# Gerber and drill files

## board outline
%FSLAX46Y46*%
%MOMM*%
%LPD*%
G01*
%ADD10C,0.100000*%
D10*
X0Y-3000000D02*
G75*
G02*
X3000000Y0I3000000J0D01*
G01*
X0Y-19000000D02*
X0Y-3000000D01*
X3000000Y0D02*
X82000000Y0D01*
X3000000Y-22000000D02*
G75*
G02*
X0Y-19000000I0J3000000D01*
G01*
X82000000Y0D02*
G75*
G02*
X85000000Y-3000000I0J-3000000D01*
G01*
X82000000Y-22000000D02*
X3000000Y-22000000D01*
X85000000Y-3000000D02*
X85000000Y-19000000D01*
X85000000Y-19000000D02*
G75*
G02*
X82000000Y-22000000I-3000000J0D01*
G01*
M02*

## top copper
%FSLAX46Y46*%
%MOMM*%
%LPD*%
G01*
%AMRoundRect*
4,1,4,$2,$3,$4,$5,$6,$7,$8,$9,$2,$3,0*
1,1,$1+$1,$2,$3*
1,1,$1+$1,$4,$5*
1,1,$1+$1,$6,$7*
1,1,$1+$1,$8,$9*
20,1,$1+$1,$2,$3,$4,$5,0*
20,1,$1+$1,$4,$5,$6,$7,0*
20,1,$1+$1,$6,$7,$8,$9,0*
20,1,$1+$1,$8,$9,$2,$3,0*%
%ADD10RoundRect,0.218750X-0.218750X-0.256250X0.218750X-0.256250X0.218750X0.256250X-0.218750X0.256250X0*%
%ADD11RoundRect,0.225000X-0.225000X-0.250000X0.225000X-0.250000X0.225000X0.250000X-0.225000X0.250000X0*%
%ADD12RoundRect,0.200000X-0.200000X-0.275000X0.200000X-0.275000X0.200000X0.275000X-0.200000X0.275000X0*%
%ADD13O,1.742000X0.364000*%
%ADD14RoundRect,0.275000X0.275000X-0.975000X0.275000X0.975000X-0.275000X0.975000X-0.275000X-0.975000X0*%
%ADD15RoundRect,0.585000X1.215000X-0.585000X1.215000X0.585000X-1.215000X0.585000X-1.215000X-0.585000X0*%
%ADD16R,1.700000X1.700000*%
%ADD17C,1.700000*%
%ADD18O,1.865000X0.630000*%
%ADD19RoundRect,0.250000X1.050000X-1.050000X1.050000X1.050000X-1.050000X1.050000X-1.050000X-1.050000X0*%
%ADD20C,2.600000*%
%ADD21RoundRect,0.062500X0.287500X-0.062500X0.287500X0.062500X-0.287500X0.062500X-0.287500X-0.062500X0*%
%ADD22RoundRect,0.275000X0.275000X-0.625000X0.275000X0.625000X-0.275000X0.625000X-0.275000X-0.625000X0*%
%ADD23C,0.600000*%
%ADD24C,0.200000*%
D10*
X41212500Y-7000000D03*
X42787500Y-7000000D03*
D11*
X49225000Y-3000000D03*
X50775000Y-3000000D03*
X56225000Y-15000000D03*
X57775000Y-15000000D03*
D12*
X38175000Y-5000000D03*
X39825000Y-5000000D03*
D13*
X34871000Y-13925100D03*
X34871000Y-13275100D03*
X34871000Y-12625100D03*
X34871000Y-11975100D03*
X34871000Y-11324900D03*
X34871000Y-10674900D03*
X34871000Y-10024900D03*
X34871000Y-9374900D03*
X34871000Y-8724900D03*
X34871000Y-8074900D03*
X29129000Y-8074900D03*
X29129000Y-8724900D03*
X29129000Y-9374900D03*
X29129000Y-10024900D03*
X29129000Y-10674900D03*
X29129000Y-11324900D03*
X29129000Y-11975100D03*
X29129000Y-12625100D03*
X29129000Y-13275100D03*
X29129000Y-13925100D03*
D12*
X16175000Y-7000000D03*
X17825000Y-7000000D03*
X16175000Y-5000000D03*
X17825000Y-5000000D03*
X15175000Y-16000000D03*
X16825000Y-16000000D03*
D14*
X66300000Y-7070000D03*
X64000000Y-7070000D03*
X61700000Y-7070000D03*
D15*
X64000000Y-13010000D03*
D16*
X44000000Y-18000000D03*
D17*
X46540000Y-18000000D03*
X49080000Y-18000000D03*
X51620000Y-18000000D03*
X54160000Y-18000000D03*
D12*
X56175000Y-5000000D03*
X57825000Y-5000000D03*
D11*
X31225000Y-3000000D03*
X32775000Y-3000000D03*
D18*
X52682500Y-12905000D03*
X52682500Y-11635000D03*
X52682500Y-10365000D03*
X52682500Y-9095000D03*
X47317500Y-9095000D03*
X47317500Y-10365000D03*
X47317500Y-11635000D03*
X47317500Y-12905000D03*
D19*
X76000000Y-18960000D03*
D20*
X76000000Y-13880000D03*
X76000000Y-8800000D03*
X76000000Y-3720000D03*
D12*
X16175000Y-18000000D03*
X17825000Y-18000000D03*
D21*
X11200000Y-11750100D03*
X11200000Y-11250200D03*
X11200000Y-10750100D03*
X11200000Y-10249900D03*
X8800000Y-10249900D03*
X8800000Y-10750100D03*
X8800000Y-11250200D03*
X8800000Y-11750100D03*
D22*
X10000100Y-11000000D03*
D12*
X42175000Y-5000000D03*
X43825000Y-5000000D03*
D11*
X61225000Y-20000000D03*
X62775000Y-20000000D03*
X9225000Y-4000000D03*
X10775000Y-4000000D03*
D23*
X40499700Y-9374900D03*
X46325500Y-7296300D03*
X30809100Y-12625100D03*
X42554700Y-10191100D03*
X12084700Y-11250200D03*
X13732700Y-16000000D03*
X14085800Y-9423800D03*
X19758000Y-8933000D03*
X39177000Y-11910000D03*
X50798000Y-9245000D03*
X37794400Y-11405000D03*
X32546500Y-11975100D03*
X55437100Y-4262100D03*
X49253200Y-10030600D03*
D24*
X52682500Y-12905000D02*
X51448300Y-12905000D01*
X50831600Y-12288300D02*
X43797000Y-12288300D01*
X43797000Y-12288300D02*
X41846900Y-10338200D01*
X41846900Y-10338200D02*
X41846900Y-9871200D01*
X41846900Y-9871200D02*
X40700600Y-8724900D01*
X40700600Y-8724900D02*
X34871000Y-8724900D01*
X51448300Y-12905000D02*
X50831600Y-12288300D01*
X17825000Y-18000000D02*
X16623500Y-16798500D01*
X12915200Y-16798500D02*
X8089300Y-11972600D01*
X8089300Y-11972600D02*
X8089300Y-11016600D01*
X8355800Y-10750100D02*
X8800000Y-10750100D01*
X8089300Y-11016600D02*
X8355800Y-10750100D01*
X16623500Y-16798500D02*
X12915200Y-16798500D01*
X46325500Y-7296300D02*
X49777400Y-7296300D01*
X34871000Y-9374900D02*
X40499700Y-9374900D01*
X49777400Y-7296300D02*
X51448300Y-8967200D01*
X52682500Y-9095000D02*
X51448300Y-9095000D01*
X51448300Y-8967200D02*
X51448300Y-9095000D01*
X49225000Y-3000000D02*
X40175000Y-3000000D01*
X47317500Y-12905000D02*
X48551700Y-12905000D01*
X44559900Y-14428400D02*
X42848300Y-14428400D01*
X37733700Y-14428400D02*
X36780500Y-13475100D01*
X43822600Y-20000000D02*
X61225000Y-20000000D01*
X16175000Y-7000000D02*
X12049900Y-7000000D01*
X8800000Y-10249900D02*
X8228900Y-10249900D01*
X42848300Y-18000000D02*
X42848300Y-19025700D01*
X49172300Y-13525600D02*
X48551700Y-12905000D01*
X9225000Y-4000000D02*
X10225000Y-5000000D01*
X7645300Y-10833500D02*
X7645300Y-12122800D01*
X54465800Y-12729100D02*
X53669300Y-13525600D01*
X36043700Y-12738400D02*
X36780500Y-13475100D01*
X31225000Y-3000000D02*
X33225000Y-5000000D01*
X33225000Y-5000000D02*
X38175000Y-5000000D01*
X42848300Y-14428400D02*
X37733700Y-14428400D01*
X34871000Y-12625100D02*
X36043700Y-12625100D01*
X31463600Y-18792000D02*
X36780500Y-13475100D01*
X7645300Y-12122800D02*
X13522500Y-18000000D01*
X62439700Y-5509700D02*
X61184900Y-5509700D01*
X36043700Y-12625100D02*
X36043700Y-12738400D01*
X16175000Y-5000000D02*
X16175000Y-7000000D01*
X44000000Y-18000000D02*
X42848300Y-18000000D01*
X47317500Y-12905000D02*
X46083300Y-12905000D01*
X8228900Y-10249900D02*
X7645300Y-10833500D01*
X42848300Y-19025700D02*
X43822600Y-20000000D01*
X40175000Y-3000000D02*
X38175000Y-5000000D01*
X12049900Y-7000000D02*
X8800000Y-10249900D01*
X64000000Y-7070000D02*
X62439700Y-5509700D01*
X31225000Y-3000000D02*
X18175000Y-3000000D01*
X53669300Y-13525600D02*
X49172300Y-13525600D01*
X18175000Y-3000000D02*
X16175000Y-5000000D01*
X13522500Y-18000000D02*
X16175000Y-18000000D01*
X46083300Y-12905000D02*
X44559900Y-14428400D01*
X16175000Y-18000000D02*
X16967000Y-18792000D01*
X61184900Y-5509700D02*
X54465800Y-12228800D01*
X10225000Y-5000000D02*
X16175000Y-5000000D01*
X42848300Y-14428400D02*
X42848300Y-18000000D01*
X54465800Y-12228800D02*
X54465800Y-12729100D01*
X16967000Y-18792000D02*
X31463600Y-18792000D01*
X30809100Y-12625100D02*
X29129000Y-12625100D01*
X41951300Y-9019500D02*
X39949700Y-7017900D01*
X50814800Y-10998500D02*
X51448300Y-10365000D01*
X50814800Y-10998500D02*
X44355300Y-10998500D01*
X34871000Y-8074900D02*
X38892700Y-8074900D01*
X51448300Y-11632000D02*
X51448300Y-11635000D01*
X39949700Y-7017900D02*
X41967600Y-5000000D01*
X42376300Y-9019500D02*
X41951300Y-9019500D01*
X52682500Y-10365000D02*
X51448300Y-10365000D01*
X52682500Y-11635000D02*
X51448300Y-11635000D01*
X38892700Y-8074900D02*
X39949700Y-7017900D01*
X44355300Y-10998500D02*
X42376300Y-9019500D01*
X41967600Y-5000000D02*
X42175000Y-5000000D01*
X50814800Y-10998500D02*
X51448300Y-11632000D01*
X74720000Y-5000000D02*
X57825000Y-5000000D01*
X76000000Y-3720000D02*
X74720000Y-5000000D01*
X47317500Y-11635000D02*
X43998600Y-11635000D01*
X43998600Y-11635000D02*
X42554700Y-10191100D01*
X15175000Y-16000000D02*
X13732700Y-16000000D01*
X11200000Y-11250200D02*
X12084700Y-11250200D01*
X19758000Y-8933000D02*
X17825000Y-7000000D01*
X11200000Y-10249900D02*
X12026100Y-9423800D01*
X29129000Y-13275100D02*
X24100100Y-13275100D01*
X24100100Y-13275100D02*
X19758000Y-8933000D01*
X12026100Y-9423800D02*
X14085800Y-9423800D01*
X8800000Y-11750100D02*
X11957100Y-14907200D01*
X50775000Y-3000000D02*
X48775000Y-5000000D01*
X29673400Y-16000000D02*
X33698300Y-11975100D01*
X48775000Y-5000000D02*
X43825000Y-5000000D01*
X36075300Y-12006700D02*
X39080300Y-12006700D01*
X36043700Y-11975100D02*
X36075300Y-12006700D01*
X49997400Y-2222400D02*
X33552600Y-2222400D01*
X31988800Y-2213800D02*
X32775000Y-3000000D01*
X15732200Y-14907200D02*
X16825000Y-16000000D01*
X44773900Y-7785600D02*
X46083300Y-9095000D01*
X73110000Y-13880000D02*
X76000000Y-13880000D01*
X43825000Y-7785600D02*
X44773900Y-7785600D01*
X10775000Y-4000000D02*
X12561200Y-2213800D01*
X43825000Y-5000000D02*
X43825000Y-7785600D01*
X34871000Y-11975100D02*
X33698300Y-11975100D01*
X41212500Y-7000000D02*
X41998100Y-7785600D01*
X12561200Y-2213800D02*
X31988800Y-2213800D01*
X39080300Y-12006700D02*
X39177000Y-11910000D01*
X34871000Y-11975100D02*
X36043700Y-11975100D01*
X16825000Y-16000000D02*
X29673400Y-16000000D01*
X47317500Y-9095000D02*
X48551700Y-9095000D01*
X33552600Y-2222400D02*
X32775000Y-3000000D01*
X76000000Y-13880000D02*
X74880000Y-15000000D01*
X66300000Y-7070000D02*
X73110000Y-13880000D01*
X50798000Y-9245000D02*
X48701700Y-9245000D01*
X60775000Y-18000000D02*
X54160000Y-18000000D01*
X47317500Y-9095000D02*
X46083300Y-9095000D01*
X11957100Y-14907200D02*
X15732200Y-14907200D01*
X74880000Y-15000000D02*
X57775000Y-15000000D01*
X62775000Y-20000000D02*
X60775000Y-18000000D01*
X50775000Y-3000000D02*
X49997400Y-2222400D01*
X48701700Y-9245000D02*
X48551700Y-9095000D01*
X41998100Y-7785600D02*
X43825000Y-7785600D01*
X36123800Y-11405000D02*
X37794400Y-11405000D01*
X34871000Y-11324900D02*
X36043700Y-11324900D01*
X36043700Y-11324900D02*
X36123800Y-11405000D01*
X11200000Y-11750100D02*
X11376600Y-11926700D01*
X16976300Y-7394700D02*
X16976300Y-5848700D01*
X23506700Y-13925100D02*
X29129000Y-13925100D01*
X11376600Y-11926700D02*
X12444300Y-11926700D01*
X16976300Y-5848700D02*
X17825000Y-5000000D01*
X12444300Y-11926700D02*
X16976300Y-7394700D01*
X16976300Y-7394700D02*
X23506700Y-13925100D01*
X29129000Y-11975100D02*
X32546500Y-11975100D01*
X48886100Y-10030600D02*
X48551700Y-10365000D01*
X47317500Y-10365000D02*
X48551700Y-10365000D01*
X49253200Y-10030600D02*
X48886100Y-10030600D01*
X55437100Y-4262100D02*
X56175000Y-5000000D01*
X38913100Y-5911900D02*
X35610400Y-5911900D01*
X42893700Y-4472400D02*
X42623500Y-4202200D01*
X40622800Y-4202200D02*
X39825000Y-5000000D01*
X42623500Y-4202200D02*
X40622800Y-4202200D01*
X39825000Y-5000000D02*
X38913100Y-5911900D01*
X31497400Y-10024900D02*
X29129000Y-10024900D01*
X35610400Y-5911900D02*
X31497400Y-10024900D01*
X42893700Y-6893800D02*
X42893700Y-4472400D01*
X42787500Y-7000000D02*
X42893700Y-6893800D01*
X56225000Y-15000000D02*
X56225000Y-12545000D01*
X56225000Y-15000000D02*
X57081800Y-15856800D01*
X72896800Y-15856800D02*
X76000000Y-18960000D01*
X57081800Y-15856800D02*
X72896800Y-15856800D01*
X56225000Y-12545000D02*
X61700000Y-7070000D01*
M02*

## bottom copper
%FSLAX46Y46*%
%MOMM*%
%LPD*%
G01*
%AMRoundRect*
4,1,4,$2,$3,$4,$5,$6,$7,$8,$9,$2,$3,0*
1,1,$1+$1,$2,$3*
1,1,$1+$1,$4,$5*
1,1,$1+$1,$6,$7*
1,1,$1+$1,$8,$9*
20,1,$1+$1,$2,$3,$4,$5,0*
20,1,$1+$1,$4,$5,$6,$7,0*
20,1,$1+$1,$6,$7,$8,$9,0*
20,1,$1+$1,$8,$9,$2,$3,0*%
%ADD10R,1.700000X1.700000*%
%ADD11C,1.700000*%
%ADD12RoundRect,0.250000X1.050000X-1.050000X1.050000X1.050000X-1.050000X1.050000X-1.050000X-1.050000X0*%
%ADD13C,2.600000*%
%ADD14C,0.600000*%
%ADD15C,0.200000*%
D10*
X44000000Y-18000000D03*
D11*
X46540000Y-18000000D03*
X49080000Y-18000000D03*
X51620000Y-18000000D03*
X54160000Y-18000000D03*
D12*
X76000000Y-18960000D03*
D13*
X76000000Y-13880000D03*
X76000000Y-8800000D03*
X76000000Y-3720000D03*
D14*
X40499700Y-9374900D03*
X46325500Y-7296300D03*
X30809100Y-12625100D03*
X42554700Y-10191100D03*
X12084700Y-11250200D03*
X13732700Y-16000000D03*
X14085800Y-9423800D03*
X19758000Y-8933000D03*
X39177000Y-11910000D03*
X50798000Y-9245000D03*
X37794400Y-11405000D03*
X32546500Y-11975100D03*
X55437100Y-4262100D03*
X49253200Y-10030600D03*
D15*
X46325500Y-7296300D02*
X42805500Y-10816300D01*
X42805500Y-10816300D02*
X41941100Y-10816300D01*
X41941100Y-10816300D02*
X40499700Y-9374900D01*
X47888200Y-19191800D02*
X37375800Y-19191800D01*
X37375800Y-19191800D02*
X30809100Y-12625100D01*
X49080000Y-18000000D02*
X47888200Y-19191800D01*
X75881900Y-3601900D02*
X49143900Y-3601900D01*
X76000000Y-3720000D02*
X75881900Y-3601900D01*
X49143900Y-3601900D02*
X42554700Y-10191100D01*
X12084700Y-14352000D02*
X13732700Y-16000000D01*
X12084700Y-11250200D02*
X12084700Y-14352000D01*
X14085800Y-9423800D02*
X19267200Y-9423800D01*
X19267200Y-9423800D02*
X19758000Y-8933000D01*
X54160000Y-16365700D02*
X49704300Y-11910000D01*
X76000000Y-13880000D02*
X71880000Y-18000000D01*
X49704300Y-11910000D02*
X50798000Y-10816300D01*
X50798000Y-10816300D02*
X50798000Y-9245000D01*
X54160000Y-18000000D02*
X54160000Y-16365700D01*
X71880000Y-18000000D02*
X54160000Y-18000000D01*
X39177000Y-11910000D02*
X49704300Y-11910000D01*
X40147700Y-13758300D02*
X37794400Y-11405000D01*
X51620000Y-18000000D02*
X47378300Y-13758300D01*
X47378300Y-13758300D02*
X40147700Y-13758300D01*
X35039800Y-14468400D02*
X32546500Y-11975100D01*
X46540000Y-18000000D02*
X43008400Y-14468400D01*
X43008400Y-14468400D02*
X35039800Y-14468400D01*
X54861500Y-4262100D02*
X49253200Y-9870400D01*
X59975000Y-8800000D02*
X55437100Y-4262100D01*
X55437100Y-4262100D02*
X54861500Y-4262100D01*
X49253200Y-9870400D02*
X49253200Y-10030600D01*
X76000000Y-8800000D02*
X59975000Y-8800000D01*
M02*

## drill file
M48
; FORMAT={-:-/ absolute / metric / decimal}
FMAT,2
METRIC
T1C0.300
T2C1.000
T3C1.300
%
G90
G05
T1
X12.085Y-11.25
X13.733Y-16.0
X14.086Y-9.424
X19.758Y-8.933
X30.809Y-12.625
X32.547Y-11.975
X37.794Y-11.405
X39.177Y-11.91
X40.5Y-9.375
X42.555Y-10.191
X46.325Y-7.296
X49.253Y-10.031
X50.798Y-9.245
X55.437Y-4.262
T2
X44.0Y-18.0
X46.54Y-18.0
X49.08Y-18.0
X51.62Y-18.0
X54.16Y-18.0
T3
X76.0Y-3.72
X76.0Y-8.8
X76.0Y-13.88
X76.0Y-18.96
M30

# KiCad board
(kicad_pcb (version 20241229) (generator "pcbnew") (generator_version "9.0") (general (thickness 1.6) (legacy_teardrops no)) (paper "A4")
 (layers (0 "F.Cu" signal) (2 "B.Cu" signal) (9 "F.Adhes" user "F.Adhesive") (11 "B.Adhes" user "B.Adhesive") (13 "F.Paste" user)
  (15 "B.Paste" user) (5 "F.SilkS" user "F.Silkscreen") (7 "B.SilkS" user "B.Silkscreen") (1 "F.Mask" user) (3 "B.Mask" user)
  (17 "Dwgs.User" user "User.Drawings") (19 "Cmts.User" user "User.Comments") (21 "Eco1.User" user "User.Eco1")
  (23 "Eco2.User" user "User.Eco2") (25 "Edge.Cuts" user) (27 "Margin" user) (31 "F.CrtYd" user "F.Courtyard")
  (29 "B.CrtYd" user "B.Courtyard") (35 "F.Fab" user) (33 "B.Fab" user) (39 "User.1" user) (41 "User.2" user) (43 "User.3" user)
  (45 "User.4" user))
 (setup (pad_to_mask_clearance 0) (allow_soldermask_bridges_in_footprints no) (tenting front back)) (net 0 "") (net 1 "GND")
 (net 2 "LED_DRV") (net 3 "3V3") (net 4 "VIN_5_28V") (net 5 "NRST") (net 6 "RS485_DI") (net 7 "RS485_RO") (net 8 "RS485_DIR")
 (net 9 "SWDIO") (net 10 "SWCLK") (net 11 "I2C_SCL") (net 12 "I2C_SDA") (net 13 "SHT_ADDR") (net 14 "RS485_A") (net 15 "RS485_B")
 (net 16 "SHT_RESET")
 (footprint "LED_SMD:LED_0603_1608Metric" (layer "F.Cu") (at 42 7)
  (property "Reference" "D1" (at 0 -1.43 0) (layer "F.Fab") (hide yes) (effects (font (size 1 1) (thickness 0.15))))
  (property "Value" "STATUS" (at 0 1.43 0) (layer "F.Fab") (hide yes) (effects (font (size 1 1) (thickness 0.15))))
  (pad "1" smd roundrect (at -0.7875 0) (size 0.875 0.95) (layers "F.Cu" "F.Mask" "F.Paste") (roundrect_rratio 0.25) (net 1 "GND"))
  (pad "2" smd roundrect (at 0.7875 0) (size 0.875 0.95) (layers "F.Cu" "F.Mask" "F.Paste") (roundrect_rratio 0.25) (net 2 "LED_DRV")))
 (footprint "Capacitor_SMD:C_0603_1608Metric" (layer "F.Cu") (at 50 3)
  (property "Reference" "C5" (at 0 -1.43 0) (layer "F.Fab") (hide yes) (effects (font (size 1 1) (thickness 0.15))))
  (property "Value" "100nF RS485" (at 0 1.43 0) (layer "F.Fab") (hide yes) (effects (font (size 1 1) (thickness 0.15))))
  (pad "1" smd roundrect (at -0.775 0) (size 0.9 0.95) (layers "F.Cu" "F.Mask" "F.Paste") (roundrect_rratio 0.25) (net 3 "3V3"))
  (pad "2" smd roundrect (at 0.775 0) (size 0.9 0.95) (layers "F.Cu" "F.Mask" "F.Paste") (roundrect_rratio 0.25) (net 1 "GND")))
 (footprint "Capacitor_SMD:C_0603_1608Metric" (layer "F.Cu") (at 57 15)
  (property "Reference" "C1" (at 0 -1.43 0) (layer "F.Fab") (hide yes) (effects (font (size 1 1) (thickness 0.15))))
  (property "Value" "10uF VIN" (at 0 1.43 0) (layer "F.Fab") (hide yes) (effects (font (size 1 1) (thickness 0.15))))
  (pad "1" smd roundrect (at -0.775 0) (size 0.9 0.95) (layers "F.Cu" "F.Mask" "F.Paste") (roundrect_rratio 0.25) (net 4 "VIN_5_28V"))
  (pad "2" smd roundrect (at 0.775 0) (size 0.9 0.95) (layers "F.Cu" "F.Mask" "F.Paste") (roundrect_rratio 0.25) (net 1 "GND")))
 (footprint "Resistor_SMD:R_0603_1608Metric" (layer "F.Cu") (at 39 5)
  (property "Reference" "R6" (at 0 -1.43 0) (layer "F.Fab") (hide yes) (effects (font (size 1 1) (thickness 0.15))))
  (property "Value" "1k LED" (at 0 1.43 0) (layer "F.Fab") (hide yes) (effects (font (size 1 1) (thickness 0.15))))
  (pad "1" smd roundrect (at -0.825 0) (size 0.8 0.95) (layers "F.Cu" "F.Mask" "F.Paste") (roundrect_rratio 0.25) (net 3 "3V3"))
  (pad "2" smd roundrect (at 0.825 0) (size 0.8 0.95) (layers "F.Cu" "F.Mask" "F.Paste") (roundrect_rratio 0.25) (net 2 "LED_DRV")))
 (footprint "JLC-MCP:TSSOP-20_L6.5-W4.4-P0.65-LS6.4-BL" (layer "F.Cu") (at 32 11 90)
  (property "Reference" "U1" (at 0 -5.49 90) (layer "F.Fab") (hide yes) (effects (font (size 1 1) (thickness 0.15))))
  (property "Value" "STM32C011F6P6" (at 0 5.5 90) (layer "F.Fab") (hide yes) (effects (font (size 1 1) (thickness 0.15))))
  (pad "1" smd oval (at -2.9251 2.871 90) (size 0.364 1.742) (layers "F.Cu" "F.Mask" "F.Paste"))
  (pad "2" smd oval (at -2.2751 2.871 90) (size 0.364 1.742) (layers "F.Cu" "F.Mask" "F.Paste"))
  (pad "3" smd oval (at -1.6251 2.871 90) (size 0.364 1.742) (layers "F.Cu" "F.Mask" "F.Paste") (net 3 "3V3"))
  (pad "4" smd oval (at -0.9751 2.871 90) (size 0.364 1.742) (layers "F.Cu" "F.Mask" "F.Paste") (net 1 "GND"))
  (pad "5" smd oval (at -0.3249 2.871 90) (size 0.364 1.742) (layers "F.Cu" "F.Mask" "F.Paste") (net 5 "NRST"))
  (pad "6" smd oval (at 0.3251 2.871 90) (size 0.364 1.742) (layers "F.Cu" "F.Mask" "F.Paste"))
  (pad "7" smd oval (at 0.9751 2.871 90) (size 0.364 1.742) (layers "F.Cu" "F.Mask" "F.Paste"))
  (pad "8" smd oval (at 1.6251 2.871 90) (size 0.364 1.742) (layers "F.Cu" "F.Mask" "F.Paste") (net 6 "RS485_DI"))
  (pad "9" smd oval (at 2.2751 2.871 90) (size 0.364 1.742) (layers "F.Cu" "F.Mask" "F.Paste") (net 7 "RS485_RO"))
  (pad "10" smd oval (at 2.9251 2.871 90) (size 0.364 1.742) (layers "F.Cu" "F.Mask" "F.Paste") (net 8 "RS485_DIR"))
  (pad "11" smd oval (at 2.9251 -2.871 90) (size 0.364 1.742) (layers "F.Cu" "F.Mask" "F.Paste"))
  (pad "12" smd oval (at 2.2751 -2.871 90) (size 0.364 1.742) (layers "F.Cu" "F.Mask" "F.Paste"))
  (pad "13" smd oval (at 1.6251 -2.871 90) (size 0.364 1.742) (layers "F.Cu" "F.Mask" "F.Paste"))
  (pad "14" smd oval (at 0.9751 -2.871 90) (size 0.364 1.742) (layers "F.Cu" "F.Mask" "F.Paste") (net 2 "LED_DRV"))
  (pad "15" smd oval (at 0.3251 -2.871 90) (size 0.364 1.742) (layers "F.Cu" "F.Mask" "F.Paste"))
  (pad "16" smd oval (at -0.3249 -2.871 90) (size 0.364 1.742) (layers "F.Cu" "F.Mask" "F.Paste"))
  (pad "17" smd oval (at -0.9751 -2.871 90) (size 0.364 1.742) (layers "F.Cu" "F.Mask" "F.Paste") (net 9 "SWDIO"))
  (pad "18" smd oval (at -1.6251 -2.871 90) (size 0.364 1.742) (layers "F.Cu" "F.Mask" "F.Paste") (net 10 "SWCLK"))
  (pad "19" smd oval (at -2.2751 -2.871 90) (size 0.364 1.742) (layers "F.Cu" "F.Mask" "F.Paste") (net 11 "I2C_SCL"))
  (pad "20" smd oval (at -2.9251 -2.871 90) (size 0.364 1.742) (layers "F.Cu" "F.Mask" "F.Paste") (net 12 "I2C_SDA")))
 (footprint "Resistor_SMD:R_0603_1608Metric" (layer "F.Cu") (at 17 7)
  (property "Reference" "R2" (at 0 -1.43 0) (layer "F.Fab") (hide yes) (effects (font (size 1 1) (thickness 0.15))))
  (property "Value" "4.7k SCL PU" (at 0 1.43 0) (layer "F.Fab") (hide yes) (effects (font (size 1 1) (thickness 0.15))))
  (pad "1" smd roundrect (at -0.825 0) (size 0.8 0.95) (layers "F.Cu" "F.Mask" "F.Paste") (roundrect_rratio 0.25) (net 3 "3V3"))
  (pad "2" smd roundrect (at 0.825 0) (size 0.8 0.95) (layers "F.Cu" "F.Mask" "F.Paste") (roundrect_rratio 0.25) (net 11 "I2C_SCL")))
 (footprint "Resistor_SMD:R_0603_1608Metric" (layer "F.Cu") (at 17 5)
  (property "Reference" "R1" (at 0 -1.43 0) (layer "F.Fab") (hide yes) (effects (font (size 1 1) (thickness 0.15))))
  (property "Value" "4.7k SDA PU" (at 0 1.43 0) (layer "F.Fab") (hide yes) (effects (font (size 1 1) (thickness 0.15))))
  (pad "1" smd roundrect (at -0.825 0) (size 0.8 0.95) (layers "F.Cu" "F.Mask" "F.Paste") (roundrect_rratio 0.25) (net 3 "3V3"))
  (pad "2" smd roundrect (at 0.825 0) (size 0.8 0.95) (layers "F.Cu" "F.Mask" "F.Paste") (roundrect_rratio 0.25) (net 12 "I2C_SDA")))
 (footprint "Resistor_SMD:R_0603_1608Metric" (layer "F.Cu") (at 16 16)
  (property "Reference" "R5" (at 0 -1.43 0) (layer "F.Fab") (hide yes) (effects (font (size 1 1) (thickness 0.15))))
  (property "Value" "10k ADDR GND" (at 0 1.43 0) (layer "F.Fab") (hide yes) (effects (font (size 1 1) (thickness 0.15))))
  (pad "1" smd roundrect (at -0.825 0) (size 0.8 0.95) (layers "F.Cu" "F.Mask" "F.Paste") (roundrect_rratio 0.25) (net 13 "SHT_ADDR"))
  (pad "2" smd roundrect (at 0.825 0) (size 0.8 0.95) (layers "F.Cu" "F.Mask" "F.Paste") (roundrect_rratio 0.25) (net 1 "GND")))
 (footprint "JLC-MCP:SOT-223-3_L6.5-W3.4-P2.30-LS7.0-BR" (layer "F.Cu") (at 64 10 90)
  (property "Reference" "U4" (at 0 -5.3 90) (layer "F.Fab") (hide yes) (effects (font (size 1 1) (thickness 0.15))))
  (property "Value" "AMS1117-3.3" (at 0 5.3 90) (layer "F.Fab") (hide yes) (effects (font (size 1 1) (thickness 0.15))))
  (pad "1" smd roundrect (at 2.93 2.3 90) (size 2.5 1.1) (layers "F.Cu" "F.Mask" "F.Paste") (roundrect_rratio 0.25) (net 1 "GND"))
  (pad "2" smd roundrect (at 2.93 0 90) (size 2.5 1.1) (layers "F.Cu" "F.Mask" "F.Paste") (roundrect_rratio 0.25) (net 3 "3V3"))
  (pad "3" smd roundrect (at 2.93 -2.3 90) (size 2.5 1.1) (layers "F.Cu" "F.Mask" "F.Paste") (roundrect_rratio 0.25) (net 4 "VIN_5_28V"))
  (pad "4" smd roundrect (at -3.01 0 90) (size 2.34 3.6) (layers "F.Cu" "F.Mask" "F.Paste") (roundrect_rratio 0.25)))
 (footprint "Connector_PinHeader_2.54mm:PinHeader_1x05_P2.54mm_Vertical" (layer "F.Cu") (at 44 18 90)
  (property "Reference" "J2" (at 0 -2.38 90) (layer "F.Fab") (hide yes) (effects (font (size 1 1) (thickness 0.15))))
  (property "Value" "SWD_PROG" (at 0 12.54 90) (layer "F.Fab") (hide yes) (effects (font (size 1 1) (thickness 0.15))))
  (pad "1" thru_hole rect (at 0 0 90) (size 1.7 1.7) (drill 1) (layers "*.Cu" "*.Mask") (remove_unused_layers no) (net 3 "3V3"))
  (pad "2" thru_hole circle (at 0 2.54 90) (size 1.7 1.7) (drill 1) (layers "*.Cu" "*.Mask") (remove_unused_layers no) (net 9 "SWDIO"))
  (pad "3" thru_hole circle (at 0 5.08 90) (size 1.7 1.7) (drill 1) (layers "*.Cu" "*.Mask") (remove_unused_layers no) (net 10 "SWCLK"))
  (pad "4" thru_hole circle (at 0 7.62 90) (size 1.7 1.7) (drill 1) (layers "*.Cu" "*.Mask") (remove_unused_layers no) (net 5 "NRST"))
  (pad "5" thru_hole circle (at 0 10.16 90) (size 1.7 1.7) (drill 1) (layers "*.Cu" "*.Mask") (remove_unused_layers no) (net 1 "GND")))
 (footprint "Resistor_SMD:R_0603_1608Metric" (layer "F.Cu") (at 57 5)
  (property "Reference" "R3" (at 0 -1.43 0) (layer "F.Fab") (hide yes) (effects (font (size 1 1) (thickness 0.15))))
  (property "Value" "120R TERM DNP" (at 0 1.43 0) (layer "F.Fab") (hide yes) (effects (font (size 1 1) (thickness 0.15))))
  (pad "1" smd roundrect (at -0.825 0) (size 0.8 0.95) (layers "F.Cu" "F.Mask" "F.Paste") (roundrect_rratio 0.25) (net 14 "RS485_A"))
  (pad "2" smd roundrect (at 0.825 0) (size 0.8 0.95) (layers "F.Cu" "F.Mask" "F.Paste") (roundrect_rratio 0.25) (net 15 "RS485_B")))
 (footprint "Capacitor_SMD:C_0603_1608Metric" (layer "F.Cu") (at 32 3)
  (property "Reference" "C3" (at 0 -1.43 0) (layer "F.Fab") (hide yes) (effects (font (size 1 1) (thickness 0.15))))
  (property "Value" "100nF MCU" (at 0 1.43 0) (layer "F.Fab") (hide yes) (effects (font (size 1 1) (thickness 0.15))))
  (pad "1" smd roundrect (at -0.775 0) (size 0.9 0.95) (layers "F.Cu" "F.Mask" "F.Paste") (roundrect_rratio 0.25) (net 3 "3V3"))
  (pad "2" smd roundrect (at 0.775 0) (size 0.9 0.95) (layers "F.Cu" "F.Mask" "F.Paste") (roundrect_rratio 0.25) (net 1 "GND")))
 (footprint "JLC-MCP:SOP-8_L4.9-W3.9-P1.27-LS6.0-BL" (layer "F.Cu") (at 50 11 90)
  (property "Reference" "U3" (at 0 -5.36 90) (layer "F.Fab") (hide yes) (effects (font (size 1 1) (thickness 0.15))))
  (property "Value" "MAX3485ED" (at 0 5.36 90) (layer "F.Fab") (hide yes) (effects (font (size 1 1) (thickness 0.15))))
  (pad "1" smd oval (at -1.905 2.6825 90) (size 0.63 1.865) (layers "F.Cu" "F.Mask" "F.Paste") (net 7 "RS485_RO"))
  (pad "2" smd oval (at -0.635 2.6825 90) (size 0.63 1.865) (layers "F.Cu" "F.Mask" "F.Paste") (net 8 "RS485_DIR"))
  (pad "3" smd oval (at 0.635 2.6825 90) (size 0.63 1.865) (layers "F.Cu" "F.Mask" "F.Paste") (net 8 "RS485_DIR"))
  (pad "4" smd oval (at 1.905 2.6825 90) (size 0.63 1.865) (layers "F.Cu" "F.Mask" "F.Paste") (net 6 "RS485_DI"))
  (pad "5" smd oval (at 1.905 -2.6825 90) (size 0.63 1.865) (layers "F.Cu" "F.Mask" "F.Paste") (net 1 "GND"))
  (pad "6" smd oval (at 0.635 -2.6825 90) (size 0.63 1.865) (layers "F.Cu" "F.Mask" "F.Paste") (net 14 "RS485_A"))
  (pad "7" smd oval (at -0.635 -2.6825 90) (size 0.63 1.865) (layers "F.Cu" "F.Mask" "F.Paste") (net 15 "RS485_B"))
  (pad "8" smd oval (at -1.905 -2.6825 90) (size 0.63 1.865) (layers "F.Cu" "F.Mask" "F.Paste") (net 3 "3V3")))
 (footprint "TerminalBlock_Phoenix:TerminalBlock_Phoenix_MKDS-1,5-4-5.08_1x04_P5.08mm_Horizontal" (layer "F.Cu") (at 76 18.96 90)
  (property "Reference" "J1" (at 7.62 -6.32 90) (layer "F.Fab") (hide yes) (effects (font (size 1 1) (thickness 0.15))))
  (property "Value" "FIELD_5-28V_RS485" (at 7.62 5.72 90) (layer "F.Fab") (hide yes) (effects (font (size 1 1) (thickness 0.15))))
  (pad "1" thru_hole roundrect (at 0 0 90) (size 2.6 2.6) (drill 1.3) (layers "*.Cu" "*.Mask") (remove_unused_layers no)
   (roundrect_rratio 0.096154) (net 4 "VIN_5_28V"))
  (pad "2" thru_hole circle (at 5.08 0 90) (size 2.6 2.6) (drill 1.3) (layers "*.Cu" "*.Mask") (remove_unused_layers no) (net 1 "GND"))
  (pad "3" thru_hole circle (at 10.16 0 90) (size 2.6 2.6) (drill 1.3) (layers "*.Cu" "*.Mask") (remove_unused_layers no) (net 14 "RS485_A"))
  (pad "4" thru_hole circle (at 15.24 0 90) (size 2.6 2.6) (drill 1.3) (layers "*.Cu" "*.Mask") (remove_unused_layers no) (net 15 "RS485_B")))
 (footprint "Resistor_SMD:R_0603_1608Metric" (layer "F.Cu") (at 17 18)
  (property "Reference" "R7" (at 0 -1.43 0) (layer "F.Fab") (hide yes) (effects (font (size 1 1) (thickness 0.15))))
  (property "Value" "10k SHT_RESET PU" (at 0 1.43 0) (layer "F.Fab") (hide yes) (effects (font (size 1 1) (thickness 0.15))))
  (pad "1" smd roundrect (at -0.825 0) (size 0.8 0.95) (layers "F.Cu" "F.Mask" "F.Paste") (roundrect_rratio 0.25) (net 3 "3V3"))
  (pad "2" smd roundrect (at 0.825 0) (size 0.8 0.95) (layers "F.Cu" "F.Mask" "F.Paste") (roundrect_rratio 0.25) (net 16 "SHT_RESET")))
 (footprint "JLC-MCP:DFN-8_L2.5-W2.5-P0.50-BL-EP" (layer "F.Cu") (at 10 11 90)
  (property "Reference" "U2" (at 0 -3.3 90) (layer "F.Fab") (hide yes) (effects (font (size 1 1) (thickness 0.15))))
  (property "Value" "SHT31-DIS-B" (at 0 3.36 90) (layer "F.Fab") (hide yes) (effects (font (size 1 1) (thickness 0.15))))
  (pad "1" smd roundrect (at -0.7501 1.2 90) (size 0.25 0.7) (layers "F.Cu" "F.Mask" "F.Paste") (roundrect_rratio 0.25) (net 12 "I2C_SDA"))
  (pad "2" smd roundrect (at -0.2502 1.2 90) (size 0.25 0.7) (layers "F.Cu" "F.Mask" "F.Paste") (roundrect_rratio 0.25) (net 13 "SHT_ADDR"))
  (pad "3" smd roundrect (at 0.2499 1.2 90) (size 0.25 0.7) (layers "F.Cu" "F.Mask" "F.Paste") (roundrect_rratio 0.25))
  (pad "4" smd roundrect (at 0.7501 1.2 90) (size 0.25 0.7) (layers "F.Cu" "F.Mask" "F.Paste") (roundrect_rratio 0.25) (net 11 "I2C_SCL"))
  (pad "5" smd roundrect (at 0.7501 -1.2 90) (size 0.25 0.7) (layers "F.Cu" "F.Mask" "F.Paste") (roundrect_rratio 0.25) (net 3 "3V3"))
  (pad "6" smd roundrect (at 0.2499 -1.2 90) (size 0.25 0.7) (layers "F.Cu" "F.Mask" "F.Paste") (roundrect_rratio 0.25) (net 16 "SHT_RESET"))
  (pad "7" smd roundrect (at -0.2502 -1.2 90) (size 0.25 0.7) (layers "F.Cu" "F.Mask" "F.Paste") (roundrect_rratio 0.25))
  (pad "8" smd roundrect (at -0.7501 -1.2 90) (size 0.25 0.7) (layers "F.Cu" "F.Mask" "F.Paste") (roundrect_rratio 0.25) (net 1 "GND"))
  (pad "9" smd roundrect (at 0 0.0001 90) (size 1.8 1.1) (layers "F.Cu" "F.Mask" "F.Paste") (roundrect_rratio 0.25)))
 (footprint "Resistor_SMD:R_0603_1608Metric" (layer "F.Cu") (at 43 5)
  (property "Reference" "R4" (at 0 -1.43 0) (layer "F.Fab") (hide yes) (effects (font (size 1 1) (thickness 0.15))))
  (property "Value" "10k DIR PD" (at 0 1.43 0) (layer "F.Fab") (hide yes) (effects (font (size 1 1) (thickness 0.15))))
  (pad "1" smd roundrect (at -0.825 0) (size 0.8 0.95) (layers "F.Cu" "F.Mask" "F.Paste") (roundrect_rratio 0.25) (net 8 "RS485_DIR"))
  (pad "2" smd roundrect (at 0.825 0) (size 0.8 0.95) (layers "F.Cu" "F.Mask" "F.Paste") (roundrect_rratio 0.25) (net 1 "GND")))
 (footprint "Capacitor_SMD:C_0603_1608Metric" (layer "F.Cu") (at 62 20)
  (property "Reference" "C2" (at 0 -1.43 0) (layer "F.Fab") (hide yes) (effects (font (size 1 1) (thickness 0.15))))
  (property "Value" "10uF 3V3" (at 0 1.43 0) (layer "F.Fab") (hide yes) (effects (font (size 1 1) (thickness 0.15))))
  (pad "1" smd roundrect (at -0.775 0) (size 0.9 0.95) (layers "F.Cu" "F.Mask" "F.Paste") (roundrect_rratio 0.25) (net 3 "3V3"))
  (pad "2" smd roundrect (at 0.775 0) (size 0.9 0.95) (layers "F.Cu" "F.Mask" "F.Paste") (roundrect_rratio 0.25) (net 1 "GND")))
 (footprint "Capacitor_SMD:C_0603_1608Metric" (layer "F.Cu") (at 10 4)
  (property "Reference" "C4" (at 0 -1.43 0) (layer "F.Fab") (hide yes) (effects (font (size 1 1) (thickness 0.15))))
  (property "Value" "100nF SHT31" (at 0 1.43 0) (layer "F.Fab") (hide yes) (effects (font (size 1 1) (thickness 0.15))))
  (pad "1" smd roundrect (at -0.775 0) (size 0.9 0.95) (layers "F.Cu" "F.Mask" "F.Paste") (roundrect_rratio 0.25) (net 3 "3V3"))
  (pad "2" smd roundrect (at 0.775 0) (size 0.9 0.95) (layers "F.Cu" "F.Mask" "F.Paste") (roundrect_rratio 0.25) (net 1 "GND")))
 (gr_arc (start 0 3) (mid 0.87868 0.87868) (end 3 0) (stroke (width 0.1) (type default)) (layer "Edge.Cuts"))
 (gr_line (start 0 19) (end 0 3) (stroke (width 0.1) (type default)) (layer "Edge.Cuts"))
 (gr_line (start 3 0) (end 82 0) (stroke (width 0.1) (type default)) (layer "Edge.Cuts"))
 (gr_arc (start 3 22) (mid 0.87868 21.12132) (end 0 19) (stroke (width 0.1) (type default)) (layer "Edge.Cuts"))
 (gr_arc (start 82 0) (mid 84.12132 0.87868) (end 85 3) (stroke (width 0.1) (type default)) (layer "Edge.Cuts"))
 (gr_line (start 82 22) (end 3 22) (stroke (width 0.1) (type default)) (layer "Edge.Cuts"))
 (gr_line (start 85 3) (end 85 19) (stroke (width 0.1) (type default)) (layer "Edge.Cuts"))
 (gr_arc (start 85 19) (mid 84.12132 21.12132) (end 82 22) (stroke (width 0.1) (type default)) (layer "Edge.Cuts"))
 (segment (start 52.6825 12.905) (end 51.4483 12.905) (width 0.2) (layer "F.Cu") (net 7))
 (segment (start 50.8316 12.2883) (end 43.797 12.2883) (width 0.2) (layer "F.Cu") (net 7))
 (segment (start 43.797 12.2883) (end 41.8469 10.3382) (width 0.2) (layer "F.Cu") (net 7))
 (segment (start 41.8469 10.3382) (end 41.8469 9.8712) (width 0.2) (layer "F.Cu") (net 7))
 (segment (start 41.8469 9.8712) (end 40.7006 8.7249) (width 0.2) (layer "F.Cu") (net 7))
 (segment (start 40.7006 8.7249) (end 34.871 8.7249) (width 0.2) (layer "F.Cu") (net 7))
 (segment (start 51.4483 12.905) (end 50.8316 12.2883) (width 0.2) (layer "F.Cu") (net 7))
 (segment (start 17.825 18) (end 16.6235 16.7985) (width 0.2) (layer "F.Cu") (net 16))
 (segment (start 12.9152 16.7985) (end 8.0893 11.9726) (width 0.2) (layer "F.Cu") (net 16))
 (segment (start 8.0893 11.9726) (end 8.0893 11.0166) (width 0.2) (layer "F.Cu") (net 16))
 (segment (start 8.3558 10.7501) (end 8.8 10.7501) (width 0.2) (layer "F.Cu") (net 16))
 (segment (start 8.0893 11.0166) (end 8.3558 10.7501) (width 0.2) (layer "F.Cu") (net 16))
 (segment (start 16.6235 16.7985) (end 12.9152 16.7985) (width 0.2) (layer "F.Cu") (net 16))
 (segment (start 46.3255 7.2963) (end 49.7774 7.2963) (width 0.2) (layer "F.Cu") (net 6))
 (segment (start 34.871 9.3749) (end 40.4997 9.3749) (width 0.2) (layer "F.Cu") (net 6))
 (segment (start 49.7774 7.2963) (end 51.4483 8.9672) (width 0.2) (layer "F.Cu") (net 6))
 (segment (start 52.6825 9.095) (end 51.4483 9.095) (width 0.2) (layer "F.Cu") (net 6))
 (segment (start 51.4483 8.9672) (end 51.4483 9.095) (width 0.2) (layer "F.Cu") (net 6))
 (via (at 40.4997 9.3749) (size 0.6) (drill 0.3) (layers "F.Cu" "B.Cu") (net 6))
 (via (at 46.3255 7.2963) (size 0.6) (drill 0.3) (layers "F.Cu" "B.Cu") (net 6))
 (segment (start 46.3255 7.2963) (end 42.8055 10.8163) (width 0.2) (layer "B.Cu") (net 6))
 (segment (start 42.8055 10.8163) (end 41.9411 10.8163) (width 0.2) (layer "B.Cu") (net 6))
 (segment (start 41.9411 10.8163) (end 40.4997 9.3749) (width 0.2) (layer "B.Cu") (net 6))
 (segment (start 49.225 3) (end 40.175 3) (width 0.2) (layer "F.Cu") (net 3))
 (segment (start 47.3175 12.905) (end 48.5517 12.905) (width 0.2) (layer "F.Cu") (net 3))
 (segment (start 44.5599 14.4284) (end 42.8483 14.4284) (width 0.2) (layer "F.Cu") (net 3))
 (segment (start 37.7337 14.4284) (end 36.7805 13.4751) (width 0.2) (layer "F.Cu") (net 3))
 (segment (start 43.8226 20) (end 61.225 20) (width 0.2) (layer "F.Cu") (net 3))
 (segment (start 16.175 7) (end 12.0499 7) (width 0.2) (layer "F.Cu") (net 3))
 (segment (start 8.8 10.2499) (end 8.2289 10.2499) (width 0.2) (layer "F.Cu") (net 3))
 (segment (start 42.8483 18) (end 42.8483 19.0257) (width 0.2) (layer "F.Cu") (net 3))
 (segment (start 49.1723 13.5256) (end 48.5517 12.905) (width 0.2) (layer "F.Cu") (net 3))
 (segment (start 9.225 4) (end 10.225 5) (width 0.2) (layer "F.Cu") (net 3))
 (segment (start 7.6453 10.8335) (end 7.6453 12.1228) (width 0.2) (layer "F.Cu") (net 3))
 (segment (start 54.4658 12.7291) (end 53.6693 13.5256) (width 0.2) (layer "F.Cu") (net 3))
 (segment (start 36.0437 12.7384) (end 36.7805 13.4751) (width 0.2) (layer "F.Cu") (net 3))
 (segment (start 31.225 3) (end 33.225 5) (width 0.2) (layer "F.Cu") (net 3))
 (segment (start 33.225 5) (end 38.175 5) (width 0.2) (layer "F.Cu") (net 3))
 (segment (start 42.8483 14.4284) (end 37.7337 14.4284) (width 0.2) (layer "F.Cu") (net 3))
 (segment (start 34.871 12.6251) (end 36.0437 12.6251) (width 0.2) (layer "F.Cu") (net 3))
 (segment (start 31.4636 18.792) (end 36.7805 13.4751) (width 0.2) (layer "F.Cu") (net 3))
 (segment (start 7.6453 12.1228) (end 13.5225 18) (width 0.2) (layer "F.Cu") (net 3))
 (segment (start 62.4397 5.5097) (end 61.1849 5.5097) (width 0.2) (layer "F.Cu") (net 3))
 (segment (start 36.0437 12.6251) (end 36.0437 12.7384) (width 0.2) (layer "F.Cu") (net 3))
 (segment (start 16.175 5) (end 16.175 7) (width 0.2) (layer "F.Cu") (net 3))
 (segment (start 44 18) (end 42.8483 18) (width 0.2) (layer "F.Cu") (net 3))
 (segment (start 47.3175 12.905) (end 46.0833 12.905) (width 0.2) (layer "F.Cu") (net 3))
 (segment (start 8.2289 10.2499) (end 7.6453 10.8335) (width 0.2) (layer "F.Cu") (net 3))
 (segment (start 42.8483 19.0257) (end 43.8226 20) (width 0.2) (layer "F.Cu") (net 3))
 (segment (start 40.175 3) (end 38.175 5) (width 0.2) (layer "F.Cu") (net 3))
 (segment (start 12.0499 7) (end 8.8 10.2499) (width 0.2) (layer "F.Cu") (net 3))
 (segment (start 64 7.07) (end 62.4397 5.5097) (width 0.2) (layer "F.Cu") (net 3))
 (segment (start 31.225 3) (end 18.175 3) (width 0.2) (layer "F.Cu") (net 3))
 (segment (start 53.6693 13.5256) (end 49.1723 13.5256) (width 0.2) (layer "F.Cu") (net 3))
 (segment (start 18.175 3) (end 16.175 5) (width 0.2) (layer "F.Cu") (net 3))
 (segment (start 13.5225 18) (end 16.175 18) (width 0.2) (layer "F.Cu") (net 3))
 (segment (start 46.0833 12.905) (end 44.5599 14.4284) (width 0.2) (layer "F.Cu") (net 3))
 (segment (start 16.175 18) (end 16.967 18.792) (width 0.2) (layer "F.Cu") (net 3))
 (segment (start 61.1849 5.5097) (end 54.4658 12.2288) (width 0.2) (layer "F.Cu") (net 3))
 (segment (start 10.225 5) (end 16.175 5) (width 0.2) (layer "F.Cu") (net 3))
 (segment (start 42.8483 14.4284) (end 42.8483 18) (width 0.2) (layer "F.Cu") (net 3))
 (segment (start 54.4658 12.2288) (end 54.4658 12.7291) (width 0.2) (layer "F.Cu") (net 3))
 (segment (start 16.967 18.792) (end 31.4636 18.792) (width 0.2) (layer "F.Cu") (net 3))
 (segment (start 30.8091 12.6251) (end 29.129 12.6251) (width 0.2) (layer "F.Cu") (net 10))
 (via (at 30.8091 12.6251) (size 0.6) (drill 0.3) (layers "F.Cu" "B.Cu") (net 10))
 (segment (start 47.8882 19.1918) (end 37.3758 19.1918) (width 0.2) (layer "B.Cu") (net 10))
 (segment (start 37.3758 19.1918) (end 30.8091 12.6251) (width 0.2) (layer "B.Cu") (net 10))
 (segment (start 49.08 18) (end 47.8882 19.1918) (width 0.2) (layer "B.Cu") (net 10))
 (segment (start 41.9513 9.0195) (end 39.9497 7.0179) (width 0.2) (layer "F.Cu") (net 8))
 (segment (start 50.8148 10.9985) (end 51.4483 10.365) (width 0.2) (layer "F.Cu") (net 8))
 (segment (start 50.8148 10.9985) (end 44.3553 10.9985) (width 0.2) (layer "F.Cu") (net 8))
 (segment (start 34.871 8.0749) (end 38.8927 8.0749) (width 0.2) (layer "F.Cu") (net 8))
 (segment (start 51.4483 11.632) (end 51.4483 11.635) (width 0.2) (layer "F.Cu") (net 8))
 (segment (start 39.9497 7.0179) (end 41.9676 5) (width 0.2) (layer "F.Cu") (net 8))
 (segment (start 42.3763 9.0195) (end 41.9513 9.0195) (width 0.2) (layer "F.Cu") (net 8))
 (segment (start 52.6825 10.365) (end 51.4483 10.365) (width 0.2) (layer "F.Cu") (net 8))
 (segment (start 52.6825 11.635) (end 51.4483 11.635) (width 0.2) (layer "F.Cu") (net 8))
 (segment (start 38.8927 8.0749) (end 39.9497 7.0179) (width 0.2) (layer "F.Cu") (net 8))
 (segment (start 44.3553 10.9985) (end 42.3763 9.0195) (width 0.2) (layer "F.Cu") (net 8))
 (segment (start 41.9676 5) (end 42.175 5) (width 0.2) (layer "F.Cu") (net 8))
 (segment (start 50.8148 10.9985) (end 51.4483 11.632) (width 0.2) (layer "F.Cu") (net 8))
 (segment (start 74.72 5) (end 57.825 5) (width 0.2) (layer "F.Cu") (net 15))
 (segment (start 76 3.72) (end 74.72 5) (width 0.2) (layer "F.Cu") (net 15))
 (segment (start 47.3175 11.635) (end 43.9986 11.635) (width 0.2) (layer "F.Cu") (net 15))
 (segment (start 43.9986 11.635) (end 42.5547 10.1911) (width 0.2) (layer "F.Cu") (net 15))
 (via (at 42.5547 10.1911) (size 0.6) (drill 0.3) (layers "F.Cu" "B.Cu") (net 15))
 (segment (start 75.8819 3.6019) (end 49.1439 3.6019) (width 0.2) (layer "B.Cu") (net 15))
 (segment (start 76 3.72) (end 75.8819 3.6019) (width 0.2) (layer "B.Cu") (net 15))
 (segment (start 49.1439 3.6019) (end 42.5547 10.1911) (width 0.2) (layer "B.Cu") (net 15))
 (segment (start 15.175 16) (end 13.7327 16) (width 0.2) (layer "F.Cu") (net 13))
 (segment (start 11.2 11.2502) (end 12.0847 11.2502) (width 0.2) (layer "F.Cu") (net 13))
 (via (at 12.0847 11.2502) (size 0.6) (drill 0.3) (layers "F.Cu" "B.Cu") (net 13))
 (via (at 13.7327 16) (size 0.6) (drill 0.3) (layers "F.Cu" "B.Cu") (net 13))
 (segment (start 12.0847 14.352) (end 13.7327 16) (width 0.2) (layer "B.Cu") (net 13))
 (segment (start 12.0847 11.2502) (end 12.0847 14.352) (width 0.2) (layer "B.Cu") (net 13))
 (segment (start 19.758 8.933) (end 17.825 7) (width 0.2) (layer "F.Cu") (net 11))
 (segment (start 11.2 10.2499) (end 12.0261 9.4238) (width 0.2) (layer "F.Cu") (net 11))
 (segment (start 29.129 13.2751) (end 24.1001 13.2751) (width 0.2) (layer "F.Cu") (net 11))
 (segment (start 24.1001 13.2751) (end 19.758 8.933) (width 0.2) (layer "F.Cu") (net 11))
 (segment (start 12.0261 9.4238) (end 14.0858 9.4238) (width 0.2) (layer "F.Cu") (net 11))
 (via (at 14.0858 9.4238) (size 0.6) (drill 0.3) (layers "F.Cu" "B.Cu") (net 11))
 (via (at 19.758 8.933) (size 0.6) (drill 0.3) (layers "F.Cu" "B.Cu") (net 11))
 (segment (start 14.0858 9.4238) (end 19.2672 9.4238) (width 0.2) (layer "B.Cu") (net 11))
 (segment (start 19.2672 9.4238) (end 19.758 8.933) (width 0.2) (layer "B.Cu") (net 11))
 (segment (start 8.8 11.7501) (end 11.9571 14.9072) (width 0.2) (layer "F.Cu") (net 1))
 (segment (start 50.775 3) (end 48.775 5) (width 0.2) (layer "F.Cu") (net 1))
 (segment (start 29.6734 16) (end 33.6983 11.9751) (width 0.2) (layer "F.Cu") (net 1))
 (segment (start 48.775 5) (end 43.825 5) (width 0.2) (layer "F.Cu") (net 1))
 (segment (start 36.0753 12.0067) (end 39.0803 12.0067) (width 0.2) (layer "F.Cu") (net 1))
 (segment (start 36.0437 11.9751) (end 36.0753 12.0067) (width 0.2) (layer "F.Cu") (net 1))
 (segment (start 49.9974 2.2224) (end 33.5526 2.2224) (width 0.2) (layer "F.Cu") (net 1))
 (segment (start 31.9888 2.2138) (end 32.775 3) (width 0.2) (layer "F.Cu") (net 1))
 (segment (start 15.7322 14.9072) (end 16.825 16) (width 0.2) (layer "F.Cu") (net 1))
 (segment (start 44.7739 7.7856) (end 46.0833 9.095) (width 0.2) (layer "F.Cu") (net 1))
 (segment (start 73.11 13.88) (end 76 13.88) (width 0.2) (layer "F.Cu") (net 1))
 (segment (start 43.825 7.7856) (end 44.7739 7.7856) (width 0.2) (layer "F.Cu") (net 1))
 (segment (start 10.775 4) (end 12.5612 2.2138) (width 0.2) (layer "F.Cu") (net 1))
 (segment (start 43.825 5) (end 43.825 7.7856) (width 0.2) (layer "F.Cu") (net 1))
 (segment (start 34.871 11.9751) (end 33.6983 11.9751) (width 0.2) (layer "F.Cu") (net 1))
 (segment (start 41.2125 7) (end 41.9981 7.7856) (width 0.2) (layer "F.Cu") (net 1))
 (segment (start 12.5612 2.2138) (end 31.9888 2.2138) (width 0.2) (layer "F.Cu") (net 1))
 (segment (start 39.0803 12.0067) (end 39.177 11.91) (width 0.2) (layer "F.Cu") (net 1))
 (segment (start 34.871 11.9751) (end 36.0437 11.9751) (width 0.2) (layer "F.Cu") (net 1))
 (segment (start 16.825 16) (end 29.6734 16) (width 0.2) (layer "F.Cu") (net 1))
 (segment (start 47.3175 9.095) (end 48.5517 9.095) (width 0.2) (layer "F.Cu") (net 1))
 (segment (start 33.5526 2.2224) (end 32.775 3) (width 0.2) (layer "F.Cu") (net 1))
 (segment (start 76 13.88) (end 74.88 15) (width 0.2) (layer "F.Cu") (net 1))
 (segment (start 66.3 7.07) (end 73.11 13.88) (width 0.2) (layer "F.Cu") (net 1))
 (segment (start 50.798 9.245) (end 48.7017 9.245) (width 0.2) (layer "F.Cu") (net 1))
 (segment (start 60.775 18) (end 54.16 18) (width 0.2) (layer "F.Cu") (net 1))
 (segment (start 47.3175 9.095) (end 46.0833 9.095) (width 0.2) (layer "F.Cu") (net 1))
 (segment (start 11.9571 14.9072) (end 15.7322 14.9072) (width 0.2) (layer "F.Cu") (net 1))
 (segment (start 74.88 15) (end 57.775 15) (width 0.2) (layer "F.Cu") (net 1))
 (segment (start 62.775 20) (end 60.775 18) (width 0.2) (layer "F.Cu") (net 1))
 (segment (start 50.775 3) (end 49.9974 2.2224) (width 0.2) (layer "F.Cu") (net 1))
 (segment (start 48.7017 9.245) (end 48.5517 9.095) (width 0.2) (layer "F.Cu") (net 1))
 (segment (start 41.9981 7.7856) (end 43.825 7.7856) (width 0.2) (layer "F.Cu") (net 1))
 (via (at 39.177 11.91) (size 0.6) (drill 0.3) (layers "F.Cu" "B.Cu") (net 1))
 (via (at 50.798 9.245) (size 0.6) (drill 0.3) (layers "F.Cu" "B.Cu") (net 1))
 (segment (start 54.16 16.3657) (end 49.7043 11.91) (width 0.2) (layer "B.Cu") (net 1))
 (segment (start 76 13.88) (end 71.88 18) (width 0.2) (layer "B.Cu") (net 1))
 (segment (start 49.7043 11.91) (end 50.798 10.8163) (width 0.2) (layer "B.Cu") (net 1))
 (segment (start 50.798 10.8163) (end 50.798 9.245) (width 0.2) (layer "B.Cu") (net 1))
 (segment (start 54.16 18) (end 54.16 16.3657) (width 0.2) (layer "B.Cu") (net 1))
 (segment (start 71.88 18) (end 54.16 18) (width 0.2) (layer "B.Cu") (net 1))
 (segment (start 39.177 11.91) (end 49.7043 11.91) (width 0.2) (layer "B.Cu") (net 1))
 (segment (start 36.1238 11.405) (end 37.7944 11.405) (width 0.2) (layer "F.Cu") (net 5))
 (segment (start 34.871 11.3249) (end 36.0437 11.3249) (width 0.2) (layer "F.Cu") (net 5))
 (segment (start 36.0437 11.3249) (end 36.1238 11.405) (width 0.2) (layer "F.Cu") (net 5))
 (via (at 37.7944 11.405) (size 0.6) (drill 0.3) (layers "F.Cu" "B.Cu") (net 5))
 (segment (start 40.1477 13.7583) (end 37.7944 11.405) (width 0.2) (layer "B.Cu") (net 5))
 (segment (start 51.62 18) (end 47.3783 13.7583) (width 0.2) (layer "B.Cu") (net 5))
 (segment (start 47.3783 13.7583) (end 40.1477 13.7583) (width 0.2) (layer "B.Cu") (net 5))
 (segment (start 11.2 11.7501) (end 11.3766 11.9267) (width 0.2) (layer "F.Cu") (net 12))
 (segment (start 16.9763 7.3947) (end 16.9763 5.8487) (width 0.2) (layer "F.Cu") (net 12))
 (segment (start 23.5067 13.9251) (end 29.129 13.9251) (width 0.2) (layer "F.Cu") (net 12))
 (segment (start 11.3766 11.9267) (end 12.4443 11.9267) (width 0.2) (layer "F.Cu") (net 12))
 (segment (start 16.9763 5.8487) (end 17.825 5) (width 0.2) (layer "F.Cu") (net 12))
 (segment (start 12.4443 11.9267) (end 16.9763 7.3947) (width 0.2) (layer "F.Cu") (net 12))
 (segment (start 16.9763 7.3947) (end 23.5067 13.9251) (width 0.2) (layer "F.Cu") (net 12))
 (segment (start 29.129 11.9751) (end 32.5465 11.9751) (width 0.2) (layer "F.Cu") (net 9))
 (via (at 32.5465 11.9751) (size 0.6) (drill 0.3) (layers "F.Cu" "B.Cu") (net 9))
 (segment (start 35.0398 14.4684) (end 32.5465 11.9751) (width 0.2) (layer "B.Cu") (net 9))
 (segment (start 46.54 18) (end 43.0084 14.4684) (width 0.2) (layer "B.Cu") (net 9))
 (segment (start 43.0084 14.4684) (end 35.0398 14.4684) (width 0.2) (layer "B.Cu") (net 9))
 (segment (start 48.8861 10.0306) (end 48.5517 10.365) (width 0.2) (layer "F.Cu") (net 14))
 (segment (start 47.3175 10.365) (end 48.5517 10.365) (width 0.2) (layer "F.Cu") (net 14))
 (segment (start 49.2532 10.0306) (end 48.8861 10.0306) (width 0.2) (layer "F.Cu") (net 14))
 (segment (start 55.4371 4.2621) (end 56.175 5) (width 0.2) (layer "F.Cu") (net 14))
 (via (at 55.4371 4.2621) (size 0.6) (drill 0.3) (layers "F.Cu" "B.Cu") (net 14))
 (via (at 49.2532 10.0306) (size 0.6) (drill 0.3) (layers "F.Cu" "B.Cu") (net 14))
 (segment (start 54.8615 4.2621) (end 49.2532 9.8704) (width 0.2) (layer "B.Cu") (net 14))
 (segment (start 59.975 8.8) (end 55.4371 4.2621) (width 0.2) (layer "B.Cu") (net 14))
 (segment (start 55.4371 4.2621) (end 54.8615 4.2621) (width 0.2) (layer "B.Cu") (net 14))
 (segment (start 49.2532 9.8704) (end 49.2532 10.0306) (width 0.2) (layer "B.Cu") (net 14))
 (segment (start 76 8.8) (end 59.975 8.8) (width 0.2) (layer "B.Cu") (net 14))
 (segment (start 38.9131 5.9119) (end 35.6104 5.9119) (width 0.2) (layer "F.Cu") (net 2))
 (segment (start 42.8937 4.4724) (end 42.6235 4.2022) (width 0.2) (layer "F.Cu") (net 2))
 (segment (start 40.6228 4.2022) (end 39.825 5) (width 0.2) (layer "F.Cu") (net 2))
 (segment (start 42.6235 4.2022) (end 40.6228 4.2022) (width 0.2) (layer "F.Cu") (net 2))
 (segment (start 39.825 5) (end 38.9131 5.9119) (width 0.2) (layer "F.Cu") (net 2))
 (segment (start 31.4974 10.0249) (end 29.129 10.0249) (width 0.2) (layer "F.Cu") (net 2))
 (segment (start 35.6104 5.9119) (end 31.4974 10.0249) (width 0.2) (layer "F.Cu") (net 2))
 (segment (start 42.8937 6.8938) (end 42.8937 4.4724) (width 0.2) (layer "F.Cu") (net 2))
 (segment (start 42.7875 7) (end 42.8937 6.8938) (width 0.2) (layer "F.Cu") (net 2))
 (segment (start 56.225 15) (end 56.225 12.545) (width 0.2) (layer "F.Cu") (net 4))
 (segment (start 56.225 15) (end 57.0818 15.8568) (width 0.2) (layer "F.Cu") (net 4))
 (segment (start 72.8968 15.8568) (end 76 18.96) (width 0.2) (layer "F.Cu") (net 4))
 (segment (start 57.0818 15.8568) (end 72.8968 15.8568) (width 0.2) (layer "F.Cu") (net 4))
 (segment (start 56.225 12.545) (end 61.7 7.07) (width 0.2) (layer "F.Cu") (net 4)))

